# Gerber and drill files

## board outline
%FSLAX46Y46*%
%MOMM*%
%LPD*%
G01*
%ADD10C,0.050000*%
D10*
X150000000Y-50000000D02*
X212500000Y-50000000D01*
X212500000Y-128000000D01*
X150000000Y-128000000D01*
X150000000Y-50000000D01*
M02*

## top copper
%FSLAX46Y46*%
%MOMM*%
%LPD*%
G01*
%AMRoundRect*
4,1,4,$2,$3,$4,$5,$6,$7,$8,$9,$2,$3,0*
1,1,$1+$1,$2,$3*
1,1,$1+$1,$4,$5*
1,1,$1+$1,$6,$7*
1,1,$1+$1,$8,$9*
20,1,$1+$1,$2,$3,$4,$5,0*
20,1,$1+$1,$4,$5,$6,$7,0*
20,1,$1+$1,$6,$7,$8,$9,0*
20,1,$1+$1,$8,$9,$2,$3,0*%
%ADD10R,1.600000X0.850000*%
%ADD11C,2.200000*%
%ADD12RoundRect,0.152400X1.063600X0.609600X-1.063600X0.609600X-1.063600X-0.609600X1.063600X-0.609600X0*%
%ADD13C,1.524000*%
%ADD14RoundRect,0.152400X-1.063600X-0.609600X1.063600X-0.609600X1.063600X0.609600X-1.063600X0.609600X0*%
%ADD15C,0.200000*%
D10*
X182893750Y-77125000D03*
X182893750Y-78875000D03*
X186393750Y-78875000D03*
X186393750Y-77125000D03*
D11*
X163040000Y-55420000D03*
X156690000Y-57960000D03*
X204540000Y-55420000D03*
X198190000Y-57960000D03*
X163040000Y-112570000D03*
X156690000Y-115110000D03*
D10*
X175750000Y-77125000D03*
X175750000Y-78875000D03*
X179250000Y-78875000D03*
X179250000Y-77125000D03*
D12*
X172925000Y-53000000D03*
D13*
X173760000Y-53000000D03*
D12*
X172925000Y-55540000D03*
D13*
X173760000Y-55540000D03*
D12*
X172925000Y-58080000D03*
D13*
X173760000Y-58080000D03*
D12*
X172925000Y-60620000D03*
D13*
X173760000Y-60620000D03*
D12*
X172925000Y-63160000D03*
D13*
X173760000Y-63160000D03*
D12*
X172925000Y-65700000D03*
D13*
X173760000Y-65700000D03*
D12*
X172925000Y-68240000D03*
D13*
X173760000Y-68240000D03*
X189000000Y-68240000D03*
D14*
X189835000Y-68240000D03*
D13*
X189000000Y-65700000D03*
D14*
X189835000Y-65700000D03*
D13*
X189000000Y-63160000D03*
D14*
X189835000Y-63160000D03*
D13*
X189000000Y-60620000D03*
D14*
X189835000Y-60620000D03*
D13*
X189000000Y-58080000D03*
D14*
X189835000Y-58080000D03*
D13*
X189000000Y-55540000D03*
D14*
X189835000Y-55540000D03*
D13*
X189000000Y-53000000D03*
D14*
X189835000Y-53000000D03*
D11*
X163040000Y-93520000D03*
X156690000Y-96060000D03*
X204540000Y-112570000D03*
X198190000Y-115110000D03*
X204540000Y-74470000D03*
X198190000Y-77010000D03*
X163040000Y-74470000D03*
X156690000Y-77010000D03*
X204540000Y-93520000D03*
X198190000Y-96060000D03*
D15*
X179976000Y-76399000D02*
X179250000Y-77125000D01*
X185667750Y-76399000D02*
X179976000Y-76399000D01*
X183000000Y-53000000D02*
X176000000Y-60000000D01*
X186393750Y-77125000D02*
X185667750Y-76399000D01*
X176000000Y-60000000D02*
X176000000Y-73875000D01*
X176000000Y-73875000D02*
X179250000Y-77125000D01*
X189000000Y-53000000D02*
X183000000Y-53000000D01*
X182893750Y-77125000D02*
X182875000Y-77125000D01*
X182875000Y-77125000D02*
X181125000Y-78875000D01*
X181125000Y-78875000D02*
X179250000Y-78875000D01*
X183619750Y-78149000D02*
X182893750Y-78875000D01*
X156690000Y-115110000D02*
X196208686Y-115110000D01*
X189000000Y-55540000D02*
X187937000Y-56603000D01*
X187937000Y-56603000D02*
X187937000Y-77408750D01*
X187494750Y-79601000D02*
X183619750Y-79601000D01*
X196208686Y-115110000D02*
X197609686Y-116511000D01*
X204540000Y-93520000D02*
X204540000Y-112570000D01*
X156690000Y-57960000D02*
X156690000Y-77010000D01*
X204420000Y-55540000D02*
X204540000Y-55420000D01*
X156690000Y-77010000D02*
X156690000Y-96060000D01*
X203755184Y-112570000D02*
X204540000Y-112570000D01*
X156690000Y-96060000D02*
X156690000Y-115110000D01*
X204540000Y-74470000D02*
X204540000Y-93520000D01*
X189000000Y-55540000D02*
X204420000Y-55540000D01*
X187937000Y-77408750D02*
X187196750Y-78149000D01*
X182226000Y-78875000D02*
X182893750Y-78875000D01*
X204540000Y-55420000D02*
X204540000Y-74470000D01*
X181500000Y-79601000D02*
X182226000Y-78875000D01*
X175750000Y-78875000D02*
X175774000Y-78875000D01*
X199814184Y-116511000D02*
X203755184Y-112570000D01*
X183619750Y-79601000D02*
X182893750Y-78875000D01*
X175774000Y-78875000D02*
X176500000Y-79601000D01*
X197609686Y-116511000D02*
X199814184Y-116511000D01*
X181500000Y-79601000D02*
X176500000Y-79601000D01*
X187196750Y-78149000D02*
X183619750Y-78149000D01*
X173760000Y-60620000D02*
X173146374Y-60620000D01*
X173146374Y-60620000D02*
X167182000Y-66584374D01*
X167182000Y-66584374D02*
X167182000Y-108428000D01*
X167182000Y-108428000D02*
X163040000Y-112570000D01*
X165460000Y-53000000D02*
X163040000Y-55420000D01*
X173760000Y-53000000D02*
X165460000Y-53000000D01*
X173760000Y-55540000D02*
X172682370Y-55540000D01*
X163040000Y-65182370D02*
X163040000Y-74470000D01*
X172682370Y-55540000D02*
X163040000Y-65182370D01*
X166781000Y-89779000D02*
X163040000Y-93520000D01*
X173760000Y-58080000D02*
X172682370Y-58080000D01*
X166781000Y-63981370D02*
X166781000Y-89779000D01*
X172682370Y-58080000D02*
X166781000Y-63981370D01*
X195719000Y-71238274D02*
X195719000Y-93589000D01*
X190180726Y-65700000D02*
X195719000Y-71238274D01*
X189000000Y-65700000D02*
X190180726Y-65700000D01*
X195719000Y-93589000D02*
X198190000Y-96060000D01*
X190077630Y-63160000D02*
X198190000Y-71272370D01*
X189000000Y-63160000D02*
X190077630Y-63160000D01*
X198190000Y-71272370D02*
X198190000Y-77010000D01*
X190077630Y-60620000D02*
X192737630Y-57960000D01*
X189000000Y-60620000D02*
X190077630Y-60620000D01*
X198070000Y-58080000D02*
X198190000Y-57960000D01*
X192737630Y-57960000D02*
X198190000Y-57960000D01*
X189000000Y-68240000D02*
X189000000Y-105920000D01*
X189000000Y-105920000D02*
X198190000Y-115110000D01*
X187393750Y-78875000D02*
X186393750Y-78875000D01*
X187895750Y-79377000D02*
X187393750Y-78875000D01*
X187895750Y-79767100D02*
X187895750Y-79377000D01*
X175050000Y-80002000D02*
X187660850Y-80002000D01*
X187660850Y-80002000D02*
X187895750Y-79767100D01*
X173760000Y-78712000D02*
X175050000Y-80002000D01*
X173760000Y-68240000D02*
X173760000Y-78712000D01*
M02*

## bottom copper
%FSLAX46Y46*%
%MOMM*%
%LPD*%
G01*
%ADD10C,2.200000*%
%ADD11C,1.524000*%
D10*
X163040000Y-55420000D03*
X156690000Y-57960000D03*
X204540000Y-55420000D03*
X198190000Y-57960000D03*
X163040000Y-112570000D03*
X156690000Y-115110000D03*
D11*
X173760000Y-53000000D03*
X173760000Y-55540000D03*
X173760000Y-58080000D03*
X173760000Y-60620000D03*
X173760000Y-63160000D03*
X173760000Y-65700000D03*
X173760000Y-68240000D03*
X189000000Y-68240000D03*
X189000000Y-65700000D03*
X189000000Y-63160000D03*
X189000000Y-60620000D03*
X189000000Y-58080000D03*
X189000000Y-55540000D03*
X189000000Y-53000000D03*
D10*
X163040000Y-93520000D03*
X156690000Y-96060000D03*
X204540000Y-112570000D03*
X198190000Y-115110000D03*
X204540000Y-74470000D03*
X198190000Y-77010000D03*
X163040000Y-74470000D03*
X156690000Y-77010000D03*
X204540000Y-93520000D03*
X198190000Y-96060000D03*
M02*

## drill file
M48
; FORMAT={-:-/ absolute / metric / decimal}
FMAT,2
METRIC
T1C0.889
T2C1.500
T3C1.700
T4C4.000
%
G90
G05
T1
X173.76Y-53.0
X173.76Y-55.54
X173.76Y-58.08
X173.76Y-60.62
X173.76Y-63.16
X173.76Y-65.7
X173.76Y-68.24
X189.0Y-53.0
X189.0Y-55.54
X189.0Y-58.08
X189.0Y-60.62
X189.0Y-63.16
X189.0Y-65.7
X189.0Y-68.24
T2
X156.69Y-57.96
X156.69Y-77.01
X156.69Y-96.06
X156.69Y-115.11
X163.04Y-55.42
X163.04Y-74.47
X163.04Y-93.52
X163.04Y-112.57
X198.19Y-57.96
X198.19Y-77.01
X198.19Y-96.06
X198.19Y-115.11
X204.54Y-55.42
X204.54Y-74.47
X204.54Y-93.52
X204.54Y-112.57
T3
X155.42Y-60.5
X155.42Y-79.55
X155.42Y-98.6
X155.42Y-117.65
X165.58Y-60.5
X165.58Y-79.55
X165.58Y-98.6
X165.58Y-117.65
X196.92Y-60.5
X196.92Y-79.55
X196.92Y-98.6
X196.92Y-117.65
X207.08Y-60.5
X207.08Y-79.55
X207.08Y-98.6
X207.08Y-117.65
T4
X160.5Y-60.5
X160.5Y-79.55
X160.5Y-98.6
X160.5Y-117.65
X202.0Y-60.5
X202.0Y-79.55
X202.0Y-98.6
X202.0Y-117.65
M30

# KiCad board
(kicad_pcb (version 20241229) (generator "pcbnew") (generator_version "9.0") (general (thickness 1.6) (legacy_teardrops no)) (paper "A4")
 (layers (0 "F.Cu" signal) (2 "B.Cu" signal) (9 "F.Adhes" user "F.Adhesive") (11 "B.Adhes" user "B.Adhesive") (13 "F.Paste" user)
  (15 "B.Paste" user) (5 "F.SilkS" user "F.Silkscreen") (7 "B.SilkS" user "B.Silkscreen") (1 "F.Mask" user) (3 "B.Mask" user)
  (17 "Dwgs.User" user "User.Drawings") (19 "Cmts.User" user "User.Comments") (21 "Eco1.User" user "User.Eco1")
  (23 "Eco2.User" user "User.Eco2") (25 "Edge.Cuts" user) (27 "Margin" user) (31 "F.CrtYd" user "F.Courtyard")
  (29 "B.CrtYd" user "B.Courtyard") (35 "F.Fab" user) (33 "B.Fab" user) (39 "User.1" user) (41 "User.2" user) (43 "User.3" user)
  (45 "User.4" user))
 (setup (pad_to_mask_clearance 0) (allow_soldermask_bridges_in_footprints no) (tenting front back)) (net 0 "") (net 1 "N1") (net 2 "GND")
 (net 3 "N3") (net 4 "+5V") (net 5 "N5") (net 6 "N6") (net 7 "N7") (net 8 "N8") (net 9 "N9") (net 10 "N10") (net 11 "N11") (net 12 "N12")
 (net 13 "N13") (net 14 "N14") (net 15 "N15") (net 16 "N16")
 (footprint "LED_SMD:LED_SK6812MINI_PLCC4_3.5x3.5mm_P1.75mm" (layer "F.Cu") (at 184.64375 78)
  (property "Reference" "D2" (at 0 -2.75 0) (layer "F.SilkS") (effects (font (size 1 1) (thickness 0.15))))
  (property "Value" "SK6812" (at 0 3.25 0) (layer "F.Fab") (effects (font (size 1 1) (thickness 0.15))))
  (pad "1" smd rect (at -1.75 -0.875) (size 1.6 0.85) (layers "F.Cu" "F.Mask" "F.Paste") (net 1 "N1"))
  (pad "2" smd rect (at -1.75 0.875) (size 1.6 0.85) (layers "F.Cu" "F.Mask" "F.Paste") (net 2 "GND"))
  (pad "3" smd rect (at 1.75 0.875) (size 1.6 0.85) (layers "F.Cu" "F.Mask" "F.Paste") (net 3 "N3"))
  (pad "4" smd rect (at 1.75 -0.875) (size 1.6 0.85) (layers "F.Cu" "F.Mask" "F.Paste") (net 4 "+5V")))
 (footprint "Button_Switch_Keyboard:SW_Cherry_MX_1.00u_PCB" (layer "F.Cu") (at 163.04 55.42)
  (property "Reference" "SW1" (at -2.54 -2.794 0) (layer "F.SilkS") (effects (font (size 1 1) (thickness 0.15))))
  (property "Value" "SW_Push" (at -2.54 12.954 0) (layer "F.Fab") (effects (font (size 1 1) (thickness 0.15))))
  (pad "" np_thru_hole circle (at -7.62 5.08) (size 1.7 1.7) (drill 1.7) (layers "*.Cu" "*.Mask"))
  (pad "" np_thru_hole circle (at -2.54 5.08) (size 4 4) (drill 4) (layers "*.Cu" "*.Mask"))
  (pad "" np_thru_hole circle (at 2.54 5.08) (size 1.7 1.7) (drill 1.7) (layers "*.Cu" "*.Mask"))
  (pad "1" thru_hole circle (at 0 0) (size 2.2 2.2) (drill 1.5) (layers "*.Cu" "*.Mask") (remove_unused_layers no) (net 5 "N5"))
  (pad "2" thru_hole circle (at -6.35 2.54) (size 2.2 2.2) (drill 1.5) (layers "*.Cu" "*.Mask") (remove_unused_layers no) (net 2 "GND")))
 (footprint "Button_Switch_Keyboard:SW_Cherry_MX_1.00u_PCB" (layer "F.Cu") (at 204.54 55.42)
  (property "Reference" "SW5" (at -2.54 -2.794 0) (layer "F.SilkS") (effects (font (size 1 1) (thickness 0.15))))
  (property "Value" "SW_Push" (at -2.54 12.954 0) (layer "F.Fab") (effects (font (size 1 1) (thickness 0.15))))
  (pad "" np_thru_hole circle (at -7.62 5.08) (size 1.7 1.7) (drill 1.7) (layers "*.Cu" "*.Mask"))
  (pad "" np_thru_hole circle (at -2.54 5.08) (size 4 4) (drill 4) (layers "*.Cu" "*.Mask"))
  (pad "" np_thru_hole circle (at 2.54 5.08) (size 1.7 1.7) (drill 1.7) (layers "*.Cu" "*.Mask"))
  (pad "1" thru_hole circle (at 0 0) (size 2.2 2.2) (drill 1.5) (layers "*.Cu" "*.Mask") (remove_unused_layers no) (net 2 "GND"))
  (pad "2" thru_hole circle (at -6.35 2.54) (size 2.2 2.2) (drill 1.5) (layers "*.Cu" "*.Mask") (remove_unused_layers no) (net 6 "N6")))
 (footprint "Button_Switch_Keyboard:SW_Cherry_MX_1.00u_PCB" (layer "F.Cu") (at 163.04 112.57)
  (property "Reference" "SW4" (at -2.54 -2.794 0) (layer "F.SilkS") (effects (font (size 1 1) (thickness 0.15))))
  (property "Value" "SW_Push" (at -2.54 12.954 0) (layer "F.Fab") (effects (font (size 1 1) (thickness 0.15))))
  (pad "" np_thru_hole circle (at -7.62 5.08) (size 1.7 1.7) (drill 1.7) (layers "*.Cu" "*.Mask"))
  (pad "" np_thru_hole circle (at -2.54 5.08) (size 4 4) (drill 4) (layers "*.Cu" "*.Mask"))
  (pad "" np_thru_hole circle (at 2.54 5.08) (size 1.7 1.7) (drill 1.7) (layers "*.Cu" "*.Mask"))
  (pad "1" thru_hole circle (at 0 0) (size 2.2 2.2) (drill 1.5) (layers "*.Cu" "*.Mask") (remove_unused_layers no) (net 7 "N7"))
  (pad "2" thru_hole circle (at -6.35 2.54) (size 2.2 2.2) (drill 1.5) (layers "*.Cu" "*.Mask") (remove_unused_layers no) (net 2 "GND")))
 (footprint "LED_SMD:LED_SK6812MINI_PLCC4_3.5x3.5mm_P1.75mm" (layer "F.Cu") (at 177.5 78)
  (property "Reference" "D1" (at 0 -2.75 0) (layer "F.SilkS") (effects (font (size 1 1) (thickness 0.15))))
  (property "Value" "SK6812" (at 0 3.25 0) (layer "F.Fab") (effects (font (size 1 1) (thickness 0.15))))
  (pad "1" smd rect (at -1.75 -0.875) (size 1.6 0.85) (layers "F.Cu" "F.Mask" "F.Paste") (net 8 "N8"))
  (pad "2" smd rect (at -1.75 0.875) (size 1.6 0.85) (layers "F.Cu" "F.Mask" "F.Paste") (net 2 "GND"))
  (pad "3" smd rect (at 1.75 0.875) (size 1.6 0.85) (layers "F.Cu" "F.Mask" "F.Paste") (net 1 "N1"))
  (pad "4" smd rect (at 1.75 -0.875) (size 1.6 0.85) (layers "F.Cu" "F.Mask" "F.Paste") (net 4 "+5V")))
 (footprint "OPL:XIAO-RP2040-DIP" (layer "F.Cu") (at 181.38 60.62)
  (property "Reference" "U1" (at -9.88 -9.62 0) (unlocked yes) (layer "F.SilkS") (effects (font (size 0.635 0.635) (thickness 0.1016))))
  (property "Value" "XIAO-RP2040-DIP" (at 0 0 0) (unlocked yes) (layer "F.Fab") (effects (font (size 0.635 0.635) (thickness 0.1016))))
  (pad "1" smd roundrect (at -8.455 -7.62 180) (size 2.432 1.524) (layers "F.Cu" "F.Mask") (roundrect_rratio 0.1) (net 5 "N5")
   (thermal_bridge_angle 45))
  (pad "1" thru_hole circle (at -7.62 -7.62 180) (size 1.524 1.524) (drill 0.889) (layers "*.Cu" "*.Mask") (remove_unused_layers no)
   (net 5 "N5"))
  (pad "2" smd roundrect (at -8.455 -5.08 180) (size 2.432 1.524) (layers "F.Cu" "F.Mask") (roundrect_rratio 0.1) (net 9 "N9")
   (thermal_bridge_angle 45))
  (pad "2" thru_hole circle (at -7.62 -5.08 180) (size 1.524 1.524) (drill 0.889) (layers "*.Cu" "*.Mask") (remove_unused_layers no)
   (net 9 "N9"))
  (pad "3" smd roundrect (at -8.455 -2.54 180) (size 2.432 1.524) (layers "F.Cu" "F.Mask") (roundrect_rratio 0.1) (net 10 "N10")
   (thermal_bridge_angle 45))
  (pad "3" thru_hole circle (at -7.62 -2.54 180) (size 1.524 1.524) (drill 0.889) (layers "*.Cu" "*.Mask") (remove_unused_layers no)
   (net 10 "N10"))
  (pad "4" smd roundrect (at -8.455 0 180) (size 2.432 1.524) (layers "F.Cu" "F.Mask") (roundrect_rratio 0.1) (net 7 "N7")
   (thermal_bridge_angle 45))
  (pad "4" thru_hole circle (at -7.62 0 180) (size 1.524 1.524) (drill 0.889) (layers "*.Cu" "*.Mask") (remove_unused_layers no)
   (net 7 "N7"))
  (pad "5" smd roundrect (at -8.455 2.54 180) (size 2.432 1.524) (layers "F.Cu" "F.Mask") (roundrect_rratio 0.1) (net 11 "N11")
   (thermal_bridge_angle 45))
  (pad "5" thru_hole circle (at -7.62 2.54 180) (size 1.524 1.524) (drill 0.889) (layers "*.Cu" "*.Mask") (remove_unused_layers no)
   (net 11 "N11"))
  (pad "6" smd roundrect (at -8.455 5.08 180) (size 2.432 1.524) (layers "F.Cu" "F.Mask") (roundrect_rratio 0.1) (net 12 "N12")
   (thermal_bridge_angle 45))
  (pad "6" thru_hole circle (at -7.62 5.08 180) (size 1.524 1.524) (drill 0.889) (layers "*.Cu" "*.Mask") (remove_unused_layers no)
   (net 12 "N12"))
  (pad "7" smd roundrect (at -8.455 7.62 180) (size 2.432 1.524) (layers "F.Cu" "F.Mask") (roundrect_rratio 0.1) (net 3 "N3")
   (thermal_bridge_angle 45))
  (pad "7" thru_hole circle (at -7.62 7.62 180) (size 1.524 1.524) (drill 0.889) (layers "*.Cu" "*.Mask") (remove_unused_layers no)
   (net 3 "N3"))
  (pad "8" thru_hole circle (at 7.62 7.62) (size 1.524 1.524) (drill 0.889) (layers "*.Cu" "*.Mask") (remove_unused_layers no)
   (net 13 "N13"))
  (pad "8" smd roundrect (at 8.455 7.62) (size 2.432 1.524) (layers "F.Cu" "F.Mask") (roundrect_rratio 0.1) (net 13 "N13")
   (thermal_bridge_angle 45))
  (pad "9" thru_hole circle (at 7.62 5.08) (size 1.524 1.524) (drill 0.889) (layers "*.Cu" "*.Mask") (remove_unused_layers no)
   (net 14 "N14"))
  (pad "9" smd roundrect (at 8.455 5.08) (size 2.432 1.524) (layers "F.Cu" "F.Mask") (roundrect_rratio 0.1) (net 14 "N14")
   (thermal_bridge_angle 45))
  (pad "10" thru_hole circle (at 7.62 2.54) (size 1.524 1.524) (drill 0.889) (layers "*.Cu" "*.Mask") (remove_unused_layers no)
   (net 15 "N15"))
  (pad "10" smd roundrect (at 8.455 2.54) (size 2.432 1.524) (layers "F.Cu" "F.Mask") (roundrect_rratio 0.1) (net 15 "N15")
   (thermal_bridge_angle 45))
  (pad "11" thru_hole circle (at 7.62 0) (size 1.524 1.524) (drill 0.889) (layers "*.Cu" "*.Mask") (remove_unused_layers no) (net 6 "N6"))
  (pad "11" smd roundrect (at 8.455 0) (size 2.432 1.524) (layers "F.Cu" "F.Mask") (roundrect_rratio 0.1) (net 6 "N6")
   (thermal_bridge_angle 45))
  (pad "12" thru_hole circle (at 7.62 -2.54) (size 1.524 1.524) (drill 0.889) (layers "*.Cu" "*.Mask") (remove_unused_layers no)
   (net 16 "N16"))
  (pad "12" smd roundrect (at 8.455 -2.54) (size 2.432 1.524) (layers "F.Cu" "F.Mask") (roundrect_rratio 0.1) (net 16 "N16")
   (thermal_bridge_angle 45))
  (pad "13" thru_hole circle (at 7.62 -5.08) (size 1.524 1.524) (drill 0.889) (layers "*.Cu" "*.Mask") (remove_unused_layers no)
   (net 2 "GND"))
  (pad "13" smd roundrect (at 8.455 -5.08) (size 2.432 1.524) (layers "F.Cu" "F.Mask") (roundrect_rratio 0.1) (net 2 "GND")
   (thermal_bridge_angle 45))
  (pad "14" thru_hole circle (at 7.62 -7.62) (size 1.524 1.524) (drill 0.889) (layers "*.Cu" "*.Mask") (remove_unused_layers no)
   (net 4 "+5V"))
  (pad "14" smd roundrect (at 8.455 -7.62) (size 2.432 1.524) (layers "F.Cu" "F.Mask") (roundrect_rratio 0.1) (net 4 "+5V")
   (thermal_bridge_angle 45)))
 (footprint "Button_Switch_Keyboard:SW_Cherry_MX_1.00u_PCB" (layer "F.Cu") (at 163.04 93.52)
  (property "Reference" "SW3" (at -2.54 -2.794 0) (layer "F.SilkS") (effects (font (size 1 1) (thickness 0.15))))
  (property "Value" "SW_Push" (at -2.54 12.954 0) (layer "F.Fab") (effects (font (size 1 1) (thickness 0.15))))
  (pad "" np_thru_hole circle (at -7.62 5.08) (size 1.7 1.7) (drill 1.7) (layers "*.Cu" "*.Mask"))
  (pad "" np_thru_hole circle (at -2.54 5.08) (size 4 4) (drill 4) (layers "*.Cu" "*.Mask"))
  (pad "" np_thru_hole circle (at 2.54 5.08) (size 1.7 1.7) (drill 1.7) (layers "*.Cu" "*.Mask"))
  (pad "1" thru_hole circle (at 0 0) (size 2.2 2.2) (drill 1.5) (layers "*.Cu" "*.Mask") (remove_unused_layers no) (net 10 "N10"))
  (pad "2" thru_hole circle (at -6.35 2.54) (size 2.2 2.2) (drill 1.5) (layers "*.Cu" "*.Mask") (remove_unused_layers no) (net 2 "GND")))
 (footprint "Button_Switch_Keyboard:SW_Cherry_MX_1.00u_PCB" (layer "F.Cu") (at 204.54 112.57)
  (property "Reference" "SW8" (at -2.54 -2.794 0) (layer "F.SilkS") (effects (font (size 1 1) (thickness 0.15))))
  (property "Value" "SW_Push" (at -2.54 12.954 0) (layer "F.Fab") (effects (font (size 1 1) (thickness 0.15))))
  (pad "" np_thru_hole circle (at -7.62 5.08) (size 1.7 1.7) (drill 1.7) (layers "*.Cu" "*.Mask"))
  (pad "" np_thru_hole circle (at -2.54 5.08) (size 4 4) (drill 4) (layers "*.Cu" "*.Mask"))
  (pad "" np_thru_hole circle (at 2.54 5.08) (size 1.7 1.7) (drill 1.7) (layers "*.Cu" "*.Mask"))
  (pad "1" thru_hole circle (at 0 0) (size 2.2 2.2) (drill 1.5) (layers "*.Cu" "*.Mask") (remove_unused_layers no) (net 2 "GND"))
  (pad "2" thru_hole circle (at -6.35 2.54) (size 2.2 2.2) (drill 1.5) (layers "*.Cu" "*.Mask") (remove_unused_layers no) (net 13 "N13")))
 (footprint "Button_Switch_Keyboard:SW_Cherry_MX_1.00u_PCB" (layer "F.Cu") (at 204.54 74.47)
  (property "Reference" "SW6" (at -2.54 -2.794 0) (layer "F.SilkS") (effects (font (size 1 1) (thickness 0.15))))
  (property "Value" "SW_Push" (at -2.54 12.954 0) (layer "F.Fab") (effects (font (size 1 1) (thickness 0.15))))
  (pad "" np_thru_hole circle (at -7.62 5.08) (size 1.7 1.7) (drill 1.7) (layers "*.Cu" "*.Mask"))
  (pad "" np_thru_hole circle (at -2.54 5.08) (size 4 4) (drill 4) (layers "*.Cu" "*.Mask"))
  (pad "" np_thru_hole circle (at 2.54 5.08) (size 1.7 1.7) (drill 1.7) (layers "*.Cu" "*.Mask"))
  (pad "1" thru_hole circle (at 0 0) (size 2.2 2.2) (drill 1.5) (layers "*.Cu" "*.Mask") (remove_unused_layers no) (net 2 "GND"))
  (pad "2" thru_hole circle (at -6.35 2.54) (size 2.2 2.2) (drill 1.5) (layers "*.Cu" "*.Mask") (remove_unused_layers no) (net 15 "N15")))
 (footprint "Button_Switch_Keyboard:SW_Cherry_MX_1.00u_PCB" (layer "F.Cu") (at 163.04 74.47)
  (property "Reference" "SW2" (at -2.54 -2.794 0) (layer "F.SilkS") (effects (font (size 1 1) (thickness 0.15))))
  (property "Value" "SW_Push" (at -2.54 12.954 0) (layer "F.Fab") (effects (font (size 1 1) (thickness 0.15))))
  (pad "" np_thru_hole circle (at -7.62 5.08) (size 1.7 1.7) (drill 1.7) (layers "*.Cu" "*.Mask"))
  (pad "" np_thru_hole circle (at -2.54 5.08) (size 4 4) (drill 4) (layers "*.Cu" "*.Mask"))
  (pad "" np_thru_hole circle (at 2.54 5.08) (size 1.7 1.7) (drill 1.7) (layers "*.Cu" "*.Mask"))
  (pad "1" thru_hole circle (at 0 0) (size 2.2 2.2) (drill 1.5) (layers "*.Cu" "*.Mask") (remove_unused_layers no) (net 9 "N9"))
  (pad "2" thru_hole circle (at -6.35 2.54) (size 2.2 2.2) (drill 1.5) (layers "*.Cu" "*.Mask") (remove_unused_layers no) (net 2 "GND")))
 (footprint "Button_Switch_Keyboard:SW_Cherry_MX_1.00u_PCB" (layer "F.Cu") (at 204.54 93.52)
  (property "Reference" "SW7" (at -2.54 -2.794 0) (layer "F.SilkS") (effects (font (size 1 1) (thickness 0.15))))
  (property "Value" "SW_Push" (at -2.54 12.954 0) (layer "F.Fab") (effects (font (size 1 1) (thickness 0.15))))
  (pad "" np_thru_hole circle (at -7.62 5.08) (size 1.7 1.7) (drill 1.7) (layers "*.Cu" "*.Mask"))
  (pad "" np_thru_hole circle (at -2.54 5.08) (size 4 4) (drill 4) (layers "*.Cu" "*.Mask"))
  (pad "" np_thru_hole circle (at 2.54 5.08) (size 1.7 1.7) (drill 1.7) (layers "*.Cu" "*.Mask"))
  (pad "1" thru_hole circle (at 0 0) (size 2.2 2.2) (drill 1.5) (layers "*.Cu" "*.Mask") (remove_unused_layers no) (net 2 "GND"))
  (pad "2" thru_hole circle (at -6.35 2.54) (size 2.2 2.2) (drill 1.5) (layers "*.Cu" "*.Mask") (remove_unused_layers no) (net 14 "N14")))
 (gr_rect (start 150 50) (end 212.5 128) (stroke (width 0.05) (type default)) (fill no) (layer "Edge.Cuts"))
 (segment (start 179.976 76.399) (end 179.25 77.125) (width 0.2) (layer "F.Cu") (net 4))
 (segment (start 185.66775 76.399) (end 179.976 76.399) (width 0.2) (layer "F.Cu") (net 4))
 (segment (start 183 53) (end 176 60) (width 0.2) (layer "F.Cu") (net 4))
 (segment (start 186.39375 77.125) (end 185.66775 76.399) (width 0.2) (layer "F.Cu") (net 4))
 (segment (start 176 60) (end 176 73.875) (width 0.2) (layer "F.Cu") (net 4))
 (segment (start 176 73.875) (end 179.25 77.125) (width 0.2) (layer "F.Cu") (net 4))
 (segment (start 189 53) (end 183 53) (width 0.2) (layer "F.Cu") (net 4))
 (segment (start 182.89375 77.125) (end 182.875 77.125) (width 0.2) (layer "F.Cu") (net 1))
 (segment (start 182.875 77.125) (end 181.125 78.875) (width 0.2) (layer "F.Cu") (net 1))
 (segment (start 181.125 78.875) (end 179.25 78.875) (width 0.2) (layer "F.Cu") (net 1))
 (segment (start 183.61975 78.149) (end 182.89375 78.875) (width 0.2) (layer "F.Cu") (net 2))
 (segment (start 156.69 115.11) (end 196.208686 115.11) (width 0.2) (layer "F.Cu") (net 2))
 (segment (start 189 55.54) (end 187.937 56.603) (width 0.2) (layer "F.Cu") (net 2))
 (segment (start 187.937 56.603) (end 187.937 77.40875) (width 0.2) (layer "F.Cu") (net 2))
 (segment (start 187.49475 79.601) (end 183.61975 79.601) (width 0.2) (layer "F.Cu") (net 2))
 (segment (start 196.208686 115.11) (end 197.609686 116.511) (width 0.2) (layer "F.Cu") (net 2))
 (segment (start 204.54 93.52) (end 204.54 112.57) (width 0.2) (layer "F.Cu") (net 2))
 (segment (start 156.69 57.96) (end 156.69 77.01) (width 0.2) (layer "F.Cu") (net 2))
 (segment (start 204.42 55.54) (end 204.54 55.42) (width 0.2) (layer "F.Cu") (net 2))
 (segment (start 156.69 77.01) (end 156.69 96.06) (width 0.2) (layer "F.Cu") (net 2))
 (segment (start 203.755184 112.57) (end 204.54 112.57) (width 0.2) (layer "F.Cu") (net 2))
 (segment (start 156.69 96.06) (end 156.69 115.11) (width 0.2) (layer "F.Cu") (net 2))
 (segment (start 204.54 74.47) (end 204.54 93.52) (width 0.2) (layer "F.Cu") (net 2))
 (segment (start 189 55.54) (end 204.42 55.54) (width 0.2) (layer "F.Cu") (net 2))
 (segment (start 187.937 77.40875) (end 187.19675 78.149) (width 0.2) (layer "F.Cu") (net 2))
 (segment (start 182.226 78.875) (end 182.89375 78.875) (width 0.2) (layer "F.Cu") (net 2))
 (segment (start 204.54 55.42) (end 204.54 74.47) (width 0.2) (layer "F.Cu") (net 2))
 (segment (start 181.5 79.601) (end 182.226 78.875) (width 0.2) (layer "F.Cu") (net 2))
 (segment (start 175.75 78.875) (end 175.774 78.875) (width 0.2) (layer "F.Cu") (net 2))
 (segment (start 199.814184 116.511) (end 203.755184 112.57) (width 0.2) (layer "F.Cu") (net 2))
 (segment (start 183.61975 79.601) (end 182.89375 78.875) (width 0.2) (layer "F.Cu") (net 2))
 (segment (start 175.774 78.875) (end 176.5 79.601) (width 0.2) (layer "F.Cu") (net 2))
 (segment (start 197.609686 116.511) (end 199.814184 116.511) (width 0.2) (layer "F.Cu") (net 2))
 (segment (start 181.5 79.601) (end 176.5 79.601) (width 0.2) (layer "F.Cu") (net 2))
 (segment (start 187.19675 78.149) (end 183.61975 78.149) (width 0.2) (layer "F.Cu") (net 2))
 (segment (start 173.76 60.62) (end 173.146374 60.62) (width 0.2) (layer "F.Cu") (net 7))
 (segment (start 173.146374 60.62) (end 167.182 66.584374) (width 0.2) (layer "F.Cu") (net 7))
 (segment (start 167.182 66.584374) (end 167.182 108.428) (width 0.2) (layer "F.Cu") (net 7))
 (segment (start 167.182 108.428) (end 163.04 112.57) (width 0.2) (layer "F.Cu") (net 7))
 (segment (start 165.46 53) (end 163.04 55.42) (width 0.2) (layer "F.Cu") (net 5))
 (segment (start 173.76 53) (end 165.46 53) (width 0.2) (layer "F.Cu") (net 5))
 (segment (start 173.76 55.54) (end 172.68237 55.54) (width 0.2) (layer "F.Cu") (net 9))
 (segment (start 163.04 65.18237) (end 163.04 74.47) (width 0.2) (layer "F.Cu") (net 9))
 (segment (start 172.68237 55.54) (end 163.04 65.18237) (width 0.2) (layer "F.Cu") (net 9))
 (segment (start 166.781 89.779) (end 163.04 93.52) (width 0.2) (layer "F.Cu") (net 10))
 (segment (start 173.76 58.08) (end 172.68237 58.08) (width 0.2) (layer "F.Cu") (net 10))
 (segment (start 166.781 63.98137) (end 166.781 89.779) (width 0.2) (layer "F.Cu") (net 10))
 (segment (start 172.68237 58.08) (end 166.781 63.98137) (width 0.2) (layer "F.Cu") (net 10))
 (segment (start 195.719 71.238274) (end 195.719 93.589) (width 0.2) (layer "F.Cu") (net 14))
 (segment (start 190.180726 65.7) (end 195.719 71.238274) (width 0.2) (layer "F.Cu") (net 14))
 (segment (start 189 65.7) (end 190.180726 65.7) (width 0.2) (layer "F.Cu") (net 14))
 (segment (start 195.719 93.589) (end 198.19 96.06) (width 0.2) (layer "F.Cu") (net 14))
 (segment (start 190.07763 63.16) (end 198.19 71.27237) (width 0.2) (layer "F.Cu") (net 15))
 (segment (start 189 63.16) (end 190.07763 63.16) (width 0.2) (layer "F.Cu") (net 15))
 (segment (start 198.19 71.27237) (end 198.19 77.01) (width 0.2) (layer "F.Cu") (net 15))
 (segment (start 190.07763 60.62) (end 192.73763 57.96) (width 0.2) (layer "F.Cu") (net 6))
 (segment (start 189 60.62) (end 190.07763 60.62) (width 0.2) (layer "F.Cu") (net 6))
 (segment (start 198.07 58.08) (end 198.19 57.96) (width 0.2) (layer "F.Cu") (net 6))
 (segment (start 192.73763 57.96) (end 198.19 57.96) (width 0.2) (layer "F.Cu") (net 6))
 (segment (start 189 68.24) (end 189 105.92) (width 0.2) (layer "F.Cu") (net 13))
 (segment (start 189 105.92) (end 198.19 115.11) (width 0.2) (layer "F.Cu") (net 13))
 (segment (start 187.39375 78.875) (end 186.39375 78.875) (width 0.2) (layer "F.Cu") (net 3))
 (segment (start 187.89575 79.377) (end 187.39375 78.875) (width 0.2) (layer "F.Cu") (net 3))
 (segment (start 187.89575 79.7671) (end 187.89575 79.377) (width 0.2) (layer "F.Cu") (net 3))
 (segment (start 175.05 80.002) (end 187.66085 80.002) (width 0.2) (layer "F.Cu") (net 3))
 (segment (start 187.66085 80.002) (end 187.89575 79.7671) (width 0.2) (layer "F.Cu") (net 3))
 (segment (start 173.76 78.712) (end 175.05 80.002) (width 0.2) (layer "F.Cu") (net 3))
 (segment (start 173.76 68.24) (end 173.76 78.712) (width 0.2) (layer "F.Cu") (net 3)))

